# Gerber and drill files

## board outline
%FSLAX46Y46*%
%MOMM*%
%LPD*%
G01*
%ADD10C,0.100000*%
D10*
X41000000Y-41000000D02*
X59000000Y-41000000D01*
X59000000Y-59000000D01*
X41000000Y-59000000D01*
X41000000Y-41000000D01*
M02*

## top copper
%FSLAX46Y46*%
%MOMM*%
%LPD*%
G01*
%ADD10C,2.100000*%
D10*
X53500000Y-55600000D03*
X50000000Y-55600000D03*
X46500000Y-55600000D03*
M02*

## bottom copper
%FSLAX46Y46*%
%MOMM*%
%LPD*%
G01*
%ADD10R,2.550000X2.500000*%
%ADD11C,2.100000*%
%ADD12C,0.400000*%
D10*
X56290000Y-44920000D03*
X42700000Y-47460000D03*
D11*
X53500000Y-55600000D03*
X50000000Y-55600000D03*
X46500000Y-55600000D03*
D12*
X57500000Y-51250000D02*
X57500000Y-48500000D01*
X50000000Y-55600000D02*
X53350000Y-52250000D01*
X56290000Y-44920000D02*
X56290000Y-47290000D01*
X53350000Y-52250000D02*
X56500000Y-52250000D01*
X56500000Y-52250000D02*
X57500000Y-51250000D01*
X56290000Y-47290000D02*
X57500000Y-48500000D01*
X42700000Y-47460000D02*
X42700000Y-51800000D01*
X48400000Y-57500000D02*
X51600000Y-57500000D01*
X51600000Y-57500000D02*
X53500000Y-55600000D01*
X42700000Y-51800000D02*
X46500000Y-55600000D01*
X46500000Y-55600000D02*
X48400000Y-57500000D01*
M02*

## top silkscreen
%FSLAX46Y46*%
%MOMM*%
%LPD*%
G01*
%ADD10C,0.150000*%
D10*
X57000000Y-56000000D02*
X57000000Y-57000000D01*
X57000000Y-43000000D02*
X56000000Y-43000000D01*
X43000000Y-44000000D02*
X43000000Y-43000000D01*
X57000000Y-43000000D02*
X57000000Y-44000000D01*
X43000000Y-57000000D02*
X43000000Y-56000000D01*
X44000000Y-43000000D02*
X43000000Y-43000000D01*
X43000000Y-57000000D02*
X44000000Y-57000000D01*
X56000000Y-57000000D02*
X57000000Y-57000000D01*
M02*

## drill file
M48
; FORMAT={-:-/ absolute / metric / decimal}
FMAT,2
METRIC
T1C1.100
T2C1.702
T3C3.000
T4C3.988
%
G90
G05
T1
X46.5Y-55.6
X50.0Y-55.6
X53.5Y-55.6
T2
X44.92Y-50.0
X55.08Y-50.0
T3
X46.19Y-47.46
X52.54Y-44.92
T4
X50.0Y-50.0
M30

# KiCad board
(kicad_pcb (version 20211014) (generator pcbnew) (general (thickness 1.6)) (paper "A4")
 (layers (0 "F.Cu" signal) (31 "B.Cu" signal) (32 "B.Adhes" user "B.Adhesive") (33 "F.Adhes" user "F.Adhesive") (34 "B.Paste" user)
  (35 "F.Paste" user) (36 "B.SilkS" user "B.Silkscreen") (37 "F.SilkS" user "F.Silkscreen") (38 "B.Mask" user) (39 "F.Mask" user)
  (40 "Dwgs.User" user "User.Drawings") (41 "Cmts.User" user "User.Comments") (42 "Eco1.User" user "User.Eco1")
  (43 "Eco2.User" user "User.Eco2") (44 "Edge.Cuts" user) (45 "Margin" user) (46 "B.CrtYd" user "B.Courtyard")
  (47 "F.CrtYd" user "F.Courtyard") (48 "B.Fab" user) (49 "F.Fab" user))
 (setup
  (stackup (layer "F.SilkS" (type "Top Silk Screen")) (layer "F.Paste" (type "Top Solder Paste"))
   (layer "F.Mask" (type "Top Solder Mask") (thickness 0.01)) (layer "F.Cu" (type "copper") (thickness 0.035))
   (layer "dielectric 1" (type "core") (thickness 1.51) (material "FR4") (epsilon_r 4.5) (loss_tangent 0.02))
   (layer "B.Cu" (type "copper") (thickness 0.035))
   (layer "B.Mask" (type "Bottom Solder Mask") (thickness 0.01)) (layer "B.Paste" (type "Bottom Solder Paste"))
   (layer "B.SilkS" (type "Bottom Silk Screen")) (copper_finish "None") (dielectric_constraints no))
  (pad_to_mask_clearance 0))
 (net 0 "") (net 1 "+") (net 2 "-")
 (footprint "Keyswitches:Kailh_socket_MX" (layer "F.Cu") (at 50 50)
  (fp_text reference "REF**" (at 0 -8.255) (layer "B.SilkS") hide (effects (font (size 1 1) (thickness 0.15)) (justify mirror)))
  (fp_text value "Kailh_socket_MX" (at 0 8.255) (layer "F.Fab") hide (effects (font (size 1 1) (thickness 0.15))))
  (fp_line (start 7 6) (end 7 7) (layer "F.SilkS") (width 0.15))
  (fp_line (start 7 -7) (end 6 -7) (layer "F.SilkS") (width 0.15))
  (fp_line (start -7 -6) (end -7 -7) (layer "F.SilkS") (width 0.15))
  (fp_line (start 7 -7) (end 7 -6) (layer "F.SilkS") (width 0.15))
  (fp_line (start -7 7) (end -7 6) (layer "F.SilkS") (width 0.15))
  (fp_line (start -6 -7) (end -7 -7) (layer "F.SilkS") (width 0.15))
  (fp_line (start -7 7) (end -6 7) (layer "F.SilkS") (width 0.15))
  (fp_line (start 6 7) (end 7 7) (layer "F.SilkS") (width 0.15))
  (pad "" np_thru_hole circle (at 2.54 -5.08) (size 3 3) (drill 3) (layers *.Cu *.Mask))
  (pad "" np_thru_hole circle (at 5.08 0) (size 1.7018 1.7018) (drill 1.7018) (layers *.Cu *.Mask))
  (pad "" np_thru_hole circle (at -5.08 0) (size 1.7018 1.7018) (drill 1.7018) (layers *.Cu *.Mask))
  (pad "" np_thru_hole circle (at -3.81 -2.54) (size 3 3) (drill 3) (layers *.Cu *.Mask))
  (pad "" np_thru_hole circle (at 0 0) (size 3.9878 3.9878) (drill 3.9878) (layers *.Cu *.Mask))
  (pad "1" smd rect (at 6.29 -5.08) (size 2.55 2.5) (layers "B.Cu" "B.Paste" "B.Mask") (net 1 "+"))
  (pad "2" smd rect (at -7.3 -2.54) (size 2.55 2.5) (layers "B.Cu" "B.Paste" "B.Mask") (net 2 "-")))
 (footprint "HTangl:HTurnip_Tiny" (layer "B.Cu") (at 42.9 55.3 180)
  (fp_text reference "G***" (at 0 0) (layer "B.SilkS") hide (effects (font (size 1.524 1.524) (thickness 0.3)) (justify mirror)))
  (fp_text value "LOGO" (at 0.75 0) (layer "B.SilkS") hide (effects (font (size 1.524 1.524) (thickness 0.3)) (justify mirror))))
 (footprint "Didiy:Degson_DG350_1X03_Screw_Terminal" (layer "B.Cu") (at 50 55.6 180)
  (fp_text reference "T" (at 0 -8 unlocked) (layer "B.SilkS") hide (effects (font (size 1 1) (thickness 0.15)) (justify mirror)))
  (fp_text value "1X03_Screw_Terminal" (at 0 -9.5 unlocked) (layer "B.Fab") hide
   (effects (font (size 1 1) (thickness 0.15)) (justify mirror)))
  (pad "1" thru_hole circle (at -3.5 0 180) (size 2.1 2.1) (drill 1.1) (layers *.Cu *.Mask) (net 2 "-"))
  (pad "2" thru_hole circle (at 0 0 180) (size 2.1 2.1) (drill 1.1) (layers *.Cu *.Mask) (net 1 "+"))
  (pad "3" thru_hole circle (at 3.5 0 180) (size 2.1 2.1) (drill 1.1) (layers *.Cu *.Mask) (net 2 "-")))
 (gr_rect (start 59 59) (end 41 41) (layer "Edge.Cuts") (width 0.1) (fill none))
 (segment (start 57.5 51.25) (end 57.5 48.5) (width 0.4) (layer "B.Cu") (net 1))
 (segment (start 50 55.6) (end 53.35 52.25) (width 0.4) (layer "B.Cu") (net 1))
 (segment (start 56.29 44.92) (end 56.29 47.29) (width 0.4) (layer "B.Cu") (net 1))
 (segment (start 53.35 52.25) (end 56.5 52.25) (width 0.4) (layer "B.Cu") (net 1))
 (segment (start 56.5 52.25) (end 57.5 51.25) (width 0.4) (layer "B.Cu") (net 1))
 (segment (start 56.29 47.29) (end 57.5 48.5) (width 0.4) (layer "B.Cu") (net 1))
 (segment (start 42.7 47.46) (end 42.7 51.8) (width 0.4) (layer "B.Cu") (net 2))
 (segment (start 48.4 57.5) (end 51.6 57.5) (width 0.4) (layer "B.Cu") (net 2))
 (segment (start 51.6 57.5) (end 53.5 55.6) (width 0.4) (layer "B.Cu") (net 2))
 (segment (start 42.7 51.8) (end 46.5 55.6) (width 0.4) (layer "B.Cu") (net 2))
 (segment (start 46.5 55.6) (end 48.4 57.5) (width 0.4) (layer "B.Cu") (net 2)))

